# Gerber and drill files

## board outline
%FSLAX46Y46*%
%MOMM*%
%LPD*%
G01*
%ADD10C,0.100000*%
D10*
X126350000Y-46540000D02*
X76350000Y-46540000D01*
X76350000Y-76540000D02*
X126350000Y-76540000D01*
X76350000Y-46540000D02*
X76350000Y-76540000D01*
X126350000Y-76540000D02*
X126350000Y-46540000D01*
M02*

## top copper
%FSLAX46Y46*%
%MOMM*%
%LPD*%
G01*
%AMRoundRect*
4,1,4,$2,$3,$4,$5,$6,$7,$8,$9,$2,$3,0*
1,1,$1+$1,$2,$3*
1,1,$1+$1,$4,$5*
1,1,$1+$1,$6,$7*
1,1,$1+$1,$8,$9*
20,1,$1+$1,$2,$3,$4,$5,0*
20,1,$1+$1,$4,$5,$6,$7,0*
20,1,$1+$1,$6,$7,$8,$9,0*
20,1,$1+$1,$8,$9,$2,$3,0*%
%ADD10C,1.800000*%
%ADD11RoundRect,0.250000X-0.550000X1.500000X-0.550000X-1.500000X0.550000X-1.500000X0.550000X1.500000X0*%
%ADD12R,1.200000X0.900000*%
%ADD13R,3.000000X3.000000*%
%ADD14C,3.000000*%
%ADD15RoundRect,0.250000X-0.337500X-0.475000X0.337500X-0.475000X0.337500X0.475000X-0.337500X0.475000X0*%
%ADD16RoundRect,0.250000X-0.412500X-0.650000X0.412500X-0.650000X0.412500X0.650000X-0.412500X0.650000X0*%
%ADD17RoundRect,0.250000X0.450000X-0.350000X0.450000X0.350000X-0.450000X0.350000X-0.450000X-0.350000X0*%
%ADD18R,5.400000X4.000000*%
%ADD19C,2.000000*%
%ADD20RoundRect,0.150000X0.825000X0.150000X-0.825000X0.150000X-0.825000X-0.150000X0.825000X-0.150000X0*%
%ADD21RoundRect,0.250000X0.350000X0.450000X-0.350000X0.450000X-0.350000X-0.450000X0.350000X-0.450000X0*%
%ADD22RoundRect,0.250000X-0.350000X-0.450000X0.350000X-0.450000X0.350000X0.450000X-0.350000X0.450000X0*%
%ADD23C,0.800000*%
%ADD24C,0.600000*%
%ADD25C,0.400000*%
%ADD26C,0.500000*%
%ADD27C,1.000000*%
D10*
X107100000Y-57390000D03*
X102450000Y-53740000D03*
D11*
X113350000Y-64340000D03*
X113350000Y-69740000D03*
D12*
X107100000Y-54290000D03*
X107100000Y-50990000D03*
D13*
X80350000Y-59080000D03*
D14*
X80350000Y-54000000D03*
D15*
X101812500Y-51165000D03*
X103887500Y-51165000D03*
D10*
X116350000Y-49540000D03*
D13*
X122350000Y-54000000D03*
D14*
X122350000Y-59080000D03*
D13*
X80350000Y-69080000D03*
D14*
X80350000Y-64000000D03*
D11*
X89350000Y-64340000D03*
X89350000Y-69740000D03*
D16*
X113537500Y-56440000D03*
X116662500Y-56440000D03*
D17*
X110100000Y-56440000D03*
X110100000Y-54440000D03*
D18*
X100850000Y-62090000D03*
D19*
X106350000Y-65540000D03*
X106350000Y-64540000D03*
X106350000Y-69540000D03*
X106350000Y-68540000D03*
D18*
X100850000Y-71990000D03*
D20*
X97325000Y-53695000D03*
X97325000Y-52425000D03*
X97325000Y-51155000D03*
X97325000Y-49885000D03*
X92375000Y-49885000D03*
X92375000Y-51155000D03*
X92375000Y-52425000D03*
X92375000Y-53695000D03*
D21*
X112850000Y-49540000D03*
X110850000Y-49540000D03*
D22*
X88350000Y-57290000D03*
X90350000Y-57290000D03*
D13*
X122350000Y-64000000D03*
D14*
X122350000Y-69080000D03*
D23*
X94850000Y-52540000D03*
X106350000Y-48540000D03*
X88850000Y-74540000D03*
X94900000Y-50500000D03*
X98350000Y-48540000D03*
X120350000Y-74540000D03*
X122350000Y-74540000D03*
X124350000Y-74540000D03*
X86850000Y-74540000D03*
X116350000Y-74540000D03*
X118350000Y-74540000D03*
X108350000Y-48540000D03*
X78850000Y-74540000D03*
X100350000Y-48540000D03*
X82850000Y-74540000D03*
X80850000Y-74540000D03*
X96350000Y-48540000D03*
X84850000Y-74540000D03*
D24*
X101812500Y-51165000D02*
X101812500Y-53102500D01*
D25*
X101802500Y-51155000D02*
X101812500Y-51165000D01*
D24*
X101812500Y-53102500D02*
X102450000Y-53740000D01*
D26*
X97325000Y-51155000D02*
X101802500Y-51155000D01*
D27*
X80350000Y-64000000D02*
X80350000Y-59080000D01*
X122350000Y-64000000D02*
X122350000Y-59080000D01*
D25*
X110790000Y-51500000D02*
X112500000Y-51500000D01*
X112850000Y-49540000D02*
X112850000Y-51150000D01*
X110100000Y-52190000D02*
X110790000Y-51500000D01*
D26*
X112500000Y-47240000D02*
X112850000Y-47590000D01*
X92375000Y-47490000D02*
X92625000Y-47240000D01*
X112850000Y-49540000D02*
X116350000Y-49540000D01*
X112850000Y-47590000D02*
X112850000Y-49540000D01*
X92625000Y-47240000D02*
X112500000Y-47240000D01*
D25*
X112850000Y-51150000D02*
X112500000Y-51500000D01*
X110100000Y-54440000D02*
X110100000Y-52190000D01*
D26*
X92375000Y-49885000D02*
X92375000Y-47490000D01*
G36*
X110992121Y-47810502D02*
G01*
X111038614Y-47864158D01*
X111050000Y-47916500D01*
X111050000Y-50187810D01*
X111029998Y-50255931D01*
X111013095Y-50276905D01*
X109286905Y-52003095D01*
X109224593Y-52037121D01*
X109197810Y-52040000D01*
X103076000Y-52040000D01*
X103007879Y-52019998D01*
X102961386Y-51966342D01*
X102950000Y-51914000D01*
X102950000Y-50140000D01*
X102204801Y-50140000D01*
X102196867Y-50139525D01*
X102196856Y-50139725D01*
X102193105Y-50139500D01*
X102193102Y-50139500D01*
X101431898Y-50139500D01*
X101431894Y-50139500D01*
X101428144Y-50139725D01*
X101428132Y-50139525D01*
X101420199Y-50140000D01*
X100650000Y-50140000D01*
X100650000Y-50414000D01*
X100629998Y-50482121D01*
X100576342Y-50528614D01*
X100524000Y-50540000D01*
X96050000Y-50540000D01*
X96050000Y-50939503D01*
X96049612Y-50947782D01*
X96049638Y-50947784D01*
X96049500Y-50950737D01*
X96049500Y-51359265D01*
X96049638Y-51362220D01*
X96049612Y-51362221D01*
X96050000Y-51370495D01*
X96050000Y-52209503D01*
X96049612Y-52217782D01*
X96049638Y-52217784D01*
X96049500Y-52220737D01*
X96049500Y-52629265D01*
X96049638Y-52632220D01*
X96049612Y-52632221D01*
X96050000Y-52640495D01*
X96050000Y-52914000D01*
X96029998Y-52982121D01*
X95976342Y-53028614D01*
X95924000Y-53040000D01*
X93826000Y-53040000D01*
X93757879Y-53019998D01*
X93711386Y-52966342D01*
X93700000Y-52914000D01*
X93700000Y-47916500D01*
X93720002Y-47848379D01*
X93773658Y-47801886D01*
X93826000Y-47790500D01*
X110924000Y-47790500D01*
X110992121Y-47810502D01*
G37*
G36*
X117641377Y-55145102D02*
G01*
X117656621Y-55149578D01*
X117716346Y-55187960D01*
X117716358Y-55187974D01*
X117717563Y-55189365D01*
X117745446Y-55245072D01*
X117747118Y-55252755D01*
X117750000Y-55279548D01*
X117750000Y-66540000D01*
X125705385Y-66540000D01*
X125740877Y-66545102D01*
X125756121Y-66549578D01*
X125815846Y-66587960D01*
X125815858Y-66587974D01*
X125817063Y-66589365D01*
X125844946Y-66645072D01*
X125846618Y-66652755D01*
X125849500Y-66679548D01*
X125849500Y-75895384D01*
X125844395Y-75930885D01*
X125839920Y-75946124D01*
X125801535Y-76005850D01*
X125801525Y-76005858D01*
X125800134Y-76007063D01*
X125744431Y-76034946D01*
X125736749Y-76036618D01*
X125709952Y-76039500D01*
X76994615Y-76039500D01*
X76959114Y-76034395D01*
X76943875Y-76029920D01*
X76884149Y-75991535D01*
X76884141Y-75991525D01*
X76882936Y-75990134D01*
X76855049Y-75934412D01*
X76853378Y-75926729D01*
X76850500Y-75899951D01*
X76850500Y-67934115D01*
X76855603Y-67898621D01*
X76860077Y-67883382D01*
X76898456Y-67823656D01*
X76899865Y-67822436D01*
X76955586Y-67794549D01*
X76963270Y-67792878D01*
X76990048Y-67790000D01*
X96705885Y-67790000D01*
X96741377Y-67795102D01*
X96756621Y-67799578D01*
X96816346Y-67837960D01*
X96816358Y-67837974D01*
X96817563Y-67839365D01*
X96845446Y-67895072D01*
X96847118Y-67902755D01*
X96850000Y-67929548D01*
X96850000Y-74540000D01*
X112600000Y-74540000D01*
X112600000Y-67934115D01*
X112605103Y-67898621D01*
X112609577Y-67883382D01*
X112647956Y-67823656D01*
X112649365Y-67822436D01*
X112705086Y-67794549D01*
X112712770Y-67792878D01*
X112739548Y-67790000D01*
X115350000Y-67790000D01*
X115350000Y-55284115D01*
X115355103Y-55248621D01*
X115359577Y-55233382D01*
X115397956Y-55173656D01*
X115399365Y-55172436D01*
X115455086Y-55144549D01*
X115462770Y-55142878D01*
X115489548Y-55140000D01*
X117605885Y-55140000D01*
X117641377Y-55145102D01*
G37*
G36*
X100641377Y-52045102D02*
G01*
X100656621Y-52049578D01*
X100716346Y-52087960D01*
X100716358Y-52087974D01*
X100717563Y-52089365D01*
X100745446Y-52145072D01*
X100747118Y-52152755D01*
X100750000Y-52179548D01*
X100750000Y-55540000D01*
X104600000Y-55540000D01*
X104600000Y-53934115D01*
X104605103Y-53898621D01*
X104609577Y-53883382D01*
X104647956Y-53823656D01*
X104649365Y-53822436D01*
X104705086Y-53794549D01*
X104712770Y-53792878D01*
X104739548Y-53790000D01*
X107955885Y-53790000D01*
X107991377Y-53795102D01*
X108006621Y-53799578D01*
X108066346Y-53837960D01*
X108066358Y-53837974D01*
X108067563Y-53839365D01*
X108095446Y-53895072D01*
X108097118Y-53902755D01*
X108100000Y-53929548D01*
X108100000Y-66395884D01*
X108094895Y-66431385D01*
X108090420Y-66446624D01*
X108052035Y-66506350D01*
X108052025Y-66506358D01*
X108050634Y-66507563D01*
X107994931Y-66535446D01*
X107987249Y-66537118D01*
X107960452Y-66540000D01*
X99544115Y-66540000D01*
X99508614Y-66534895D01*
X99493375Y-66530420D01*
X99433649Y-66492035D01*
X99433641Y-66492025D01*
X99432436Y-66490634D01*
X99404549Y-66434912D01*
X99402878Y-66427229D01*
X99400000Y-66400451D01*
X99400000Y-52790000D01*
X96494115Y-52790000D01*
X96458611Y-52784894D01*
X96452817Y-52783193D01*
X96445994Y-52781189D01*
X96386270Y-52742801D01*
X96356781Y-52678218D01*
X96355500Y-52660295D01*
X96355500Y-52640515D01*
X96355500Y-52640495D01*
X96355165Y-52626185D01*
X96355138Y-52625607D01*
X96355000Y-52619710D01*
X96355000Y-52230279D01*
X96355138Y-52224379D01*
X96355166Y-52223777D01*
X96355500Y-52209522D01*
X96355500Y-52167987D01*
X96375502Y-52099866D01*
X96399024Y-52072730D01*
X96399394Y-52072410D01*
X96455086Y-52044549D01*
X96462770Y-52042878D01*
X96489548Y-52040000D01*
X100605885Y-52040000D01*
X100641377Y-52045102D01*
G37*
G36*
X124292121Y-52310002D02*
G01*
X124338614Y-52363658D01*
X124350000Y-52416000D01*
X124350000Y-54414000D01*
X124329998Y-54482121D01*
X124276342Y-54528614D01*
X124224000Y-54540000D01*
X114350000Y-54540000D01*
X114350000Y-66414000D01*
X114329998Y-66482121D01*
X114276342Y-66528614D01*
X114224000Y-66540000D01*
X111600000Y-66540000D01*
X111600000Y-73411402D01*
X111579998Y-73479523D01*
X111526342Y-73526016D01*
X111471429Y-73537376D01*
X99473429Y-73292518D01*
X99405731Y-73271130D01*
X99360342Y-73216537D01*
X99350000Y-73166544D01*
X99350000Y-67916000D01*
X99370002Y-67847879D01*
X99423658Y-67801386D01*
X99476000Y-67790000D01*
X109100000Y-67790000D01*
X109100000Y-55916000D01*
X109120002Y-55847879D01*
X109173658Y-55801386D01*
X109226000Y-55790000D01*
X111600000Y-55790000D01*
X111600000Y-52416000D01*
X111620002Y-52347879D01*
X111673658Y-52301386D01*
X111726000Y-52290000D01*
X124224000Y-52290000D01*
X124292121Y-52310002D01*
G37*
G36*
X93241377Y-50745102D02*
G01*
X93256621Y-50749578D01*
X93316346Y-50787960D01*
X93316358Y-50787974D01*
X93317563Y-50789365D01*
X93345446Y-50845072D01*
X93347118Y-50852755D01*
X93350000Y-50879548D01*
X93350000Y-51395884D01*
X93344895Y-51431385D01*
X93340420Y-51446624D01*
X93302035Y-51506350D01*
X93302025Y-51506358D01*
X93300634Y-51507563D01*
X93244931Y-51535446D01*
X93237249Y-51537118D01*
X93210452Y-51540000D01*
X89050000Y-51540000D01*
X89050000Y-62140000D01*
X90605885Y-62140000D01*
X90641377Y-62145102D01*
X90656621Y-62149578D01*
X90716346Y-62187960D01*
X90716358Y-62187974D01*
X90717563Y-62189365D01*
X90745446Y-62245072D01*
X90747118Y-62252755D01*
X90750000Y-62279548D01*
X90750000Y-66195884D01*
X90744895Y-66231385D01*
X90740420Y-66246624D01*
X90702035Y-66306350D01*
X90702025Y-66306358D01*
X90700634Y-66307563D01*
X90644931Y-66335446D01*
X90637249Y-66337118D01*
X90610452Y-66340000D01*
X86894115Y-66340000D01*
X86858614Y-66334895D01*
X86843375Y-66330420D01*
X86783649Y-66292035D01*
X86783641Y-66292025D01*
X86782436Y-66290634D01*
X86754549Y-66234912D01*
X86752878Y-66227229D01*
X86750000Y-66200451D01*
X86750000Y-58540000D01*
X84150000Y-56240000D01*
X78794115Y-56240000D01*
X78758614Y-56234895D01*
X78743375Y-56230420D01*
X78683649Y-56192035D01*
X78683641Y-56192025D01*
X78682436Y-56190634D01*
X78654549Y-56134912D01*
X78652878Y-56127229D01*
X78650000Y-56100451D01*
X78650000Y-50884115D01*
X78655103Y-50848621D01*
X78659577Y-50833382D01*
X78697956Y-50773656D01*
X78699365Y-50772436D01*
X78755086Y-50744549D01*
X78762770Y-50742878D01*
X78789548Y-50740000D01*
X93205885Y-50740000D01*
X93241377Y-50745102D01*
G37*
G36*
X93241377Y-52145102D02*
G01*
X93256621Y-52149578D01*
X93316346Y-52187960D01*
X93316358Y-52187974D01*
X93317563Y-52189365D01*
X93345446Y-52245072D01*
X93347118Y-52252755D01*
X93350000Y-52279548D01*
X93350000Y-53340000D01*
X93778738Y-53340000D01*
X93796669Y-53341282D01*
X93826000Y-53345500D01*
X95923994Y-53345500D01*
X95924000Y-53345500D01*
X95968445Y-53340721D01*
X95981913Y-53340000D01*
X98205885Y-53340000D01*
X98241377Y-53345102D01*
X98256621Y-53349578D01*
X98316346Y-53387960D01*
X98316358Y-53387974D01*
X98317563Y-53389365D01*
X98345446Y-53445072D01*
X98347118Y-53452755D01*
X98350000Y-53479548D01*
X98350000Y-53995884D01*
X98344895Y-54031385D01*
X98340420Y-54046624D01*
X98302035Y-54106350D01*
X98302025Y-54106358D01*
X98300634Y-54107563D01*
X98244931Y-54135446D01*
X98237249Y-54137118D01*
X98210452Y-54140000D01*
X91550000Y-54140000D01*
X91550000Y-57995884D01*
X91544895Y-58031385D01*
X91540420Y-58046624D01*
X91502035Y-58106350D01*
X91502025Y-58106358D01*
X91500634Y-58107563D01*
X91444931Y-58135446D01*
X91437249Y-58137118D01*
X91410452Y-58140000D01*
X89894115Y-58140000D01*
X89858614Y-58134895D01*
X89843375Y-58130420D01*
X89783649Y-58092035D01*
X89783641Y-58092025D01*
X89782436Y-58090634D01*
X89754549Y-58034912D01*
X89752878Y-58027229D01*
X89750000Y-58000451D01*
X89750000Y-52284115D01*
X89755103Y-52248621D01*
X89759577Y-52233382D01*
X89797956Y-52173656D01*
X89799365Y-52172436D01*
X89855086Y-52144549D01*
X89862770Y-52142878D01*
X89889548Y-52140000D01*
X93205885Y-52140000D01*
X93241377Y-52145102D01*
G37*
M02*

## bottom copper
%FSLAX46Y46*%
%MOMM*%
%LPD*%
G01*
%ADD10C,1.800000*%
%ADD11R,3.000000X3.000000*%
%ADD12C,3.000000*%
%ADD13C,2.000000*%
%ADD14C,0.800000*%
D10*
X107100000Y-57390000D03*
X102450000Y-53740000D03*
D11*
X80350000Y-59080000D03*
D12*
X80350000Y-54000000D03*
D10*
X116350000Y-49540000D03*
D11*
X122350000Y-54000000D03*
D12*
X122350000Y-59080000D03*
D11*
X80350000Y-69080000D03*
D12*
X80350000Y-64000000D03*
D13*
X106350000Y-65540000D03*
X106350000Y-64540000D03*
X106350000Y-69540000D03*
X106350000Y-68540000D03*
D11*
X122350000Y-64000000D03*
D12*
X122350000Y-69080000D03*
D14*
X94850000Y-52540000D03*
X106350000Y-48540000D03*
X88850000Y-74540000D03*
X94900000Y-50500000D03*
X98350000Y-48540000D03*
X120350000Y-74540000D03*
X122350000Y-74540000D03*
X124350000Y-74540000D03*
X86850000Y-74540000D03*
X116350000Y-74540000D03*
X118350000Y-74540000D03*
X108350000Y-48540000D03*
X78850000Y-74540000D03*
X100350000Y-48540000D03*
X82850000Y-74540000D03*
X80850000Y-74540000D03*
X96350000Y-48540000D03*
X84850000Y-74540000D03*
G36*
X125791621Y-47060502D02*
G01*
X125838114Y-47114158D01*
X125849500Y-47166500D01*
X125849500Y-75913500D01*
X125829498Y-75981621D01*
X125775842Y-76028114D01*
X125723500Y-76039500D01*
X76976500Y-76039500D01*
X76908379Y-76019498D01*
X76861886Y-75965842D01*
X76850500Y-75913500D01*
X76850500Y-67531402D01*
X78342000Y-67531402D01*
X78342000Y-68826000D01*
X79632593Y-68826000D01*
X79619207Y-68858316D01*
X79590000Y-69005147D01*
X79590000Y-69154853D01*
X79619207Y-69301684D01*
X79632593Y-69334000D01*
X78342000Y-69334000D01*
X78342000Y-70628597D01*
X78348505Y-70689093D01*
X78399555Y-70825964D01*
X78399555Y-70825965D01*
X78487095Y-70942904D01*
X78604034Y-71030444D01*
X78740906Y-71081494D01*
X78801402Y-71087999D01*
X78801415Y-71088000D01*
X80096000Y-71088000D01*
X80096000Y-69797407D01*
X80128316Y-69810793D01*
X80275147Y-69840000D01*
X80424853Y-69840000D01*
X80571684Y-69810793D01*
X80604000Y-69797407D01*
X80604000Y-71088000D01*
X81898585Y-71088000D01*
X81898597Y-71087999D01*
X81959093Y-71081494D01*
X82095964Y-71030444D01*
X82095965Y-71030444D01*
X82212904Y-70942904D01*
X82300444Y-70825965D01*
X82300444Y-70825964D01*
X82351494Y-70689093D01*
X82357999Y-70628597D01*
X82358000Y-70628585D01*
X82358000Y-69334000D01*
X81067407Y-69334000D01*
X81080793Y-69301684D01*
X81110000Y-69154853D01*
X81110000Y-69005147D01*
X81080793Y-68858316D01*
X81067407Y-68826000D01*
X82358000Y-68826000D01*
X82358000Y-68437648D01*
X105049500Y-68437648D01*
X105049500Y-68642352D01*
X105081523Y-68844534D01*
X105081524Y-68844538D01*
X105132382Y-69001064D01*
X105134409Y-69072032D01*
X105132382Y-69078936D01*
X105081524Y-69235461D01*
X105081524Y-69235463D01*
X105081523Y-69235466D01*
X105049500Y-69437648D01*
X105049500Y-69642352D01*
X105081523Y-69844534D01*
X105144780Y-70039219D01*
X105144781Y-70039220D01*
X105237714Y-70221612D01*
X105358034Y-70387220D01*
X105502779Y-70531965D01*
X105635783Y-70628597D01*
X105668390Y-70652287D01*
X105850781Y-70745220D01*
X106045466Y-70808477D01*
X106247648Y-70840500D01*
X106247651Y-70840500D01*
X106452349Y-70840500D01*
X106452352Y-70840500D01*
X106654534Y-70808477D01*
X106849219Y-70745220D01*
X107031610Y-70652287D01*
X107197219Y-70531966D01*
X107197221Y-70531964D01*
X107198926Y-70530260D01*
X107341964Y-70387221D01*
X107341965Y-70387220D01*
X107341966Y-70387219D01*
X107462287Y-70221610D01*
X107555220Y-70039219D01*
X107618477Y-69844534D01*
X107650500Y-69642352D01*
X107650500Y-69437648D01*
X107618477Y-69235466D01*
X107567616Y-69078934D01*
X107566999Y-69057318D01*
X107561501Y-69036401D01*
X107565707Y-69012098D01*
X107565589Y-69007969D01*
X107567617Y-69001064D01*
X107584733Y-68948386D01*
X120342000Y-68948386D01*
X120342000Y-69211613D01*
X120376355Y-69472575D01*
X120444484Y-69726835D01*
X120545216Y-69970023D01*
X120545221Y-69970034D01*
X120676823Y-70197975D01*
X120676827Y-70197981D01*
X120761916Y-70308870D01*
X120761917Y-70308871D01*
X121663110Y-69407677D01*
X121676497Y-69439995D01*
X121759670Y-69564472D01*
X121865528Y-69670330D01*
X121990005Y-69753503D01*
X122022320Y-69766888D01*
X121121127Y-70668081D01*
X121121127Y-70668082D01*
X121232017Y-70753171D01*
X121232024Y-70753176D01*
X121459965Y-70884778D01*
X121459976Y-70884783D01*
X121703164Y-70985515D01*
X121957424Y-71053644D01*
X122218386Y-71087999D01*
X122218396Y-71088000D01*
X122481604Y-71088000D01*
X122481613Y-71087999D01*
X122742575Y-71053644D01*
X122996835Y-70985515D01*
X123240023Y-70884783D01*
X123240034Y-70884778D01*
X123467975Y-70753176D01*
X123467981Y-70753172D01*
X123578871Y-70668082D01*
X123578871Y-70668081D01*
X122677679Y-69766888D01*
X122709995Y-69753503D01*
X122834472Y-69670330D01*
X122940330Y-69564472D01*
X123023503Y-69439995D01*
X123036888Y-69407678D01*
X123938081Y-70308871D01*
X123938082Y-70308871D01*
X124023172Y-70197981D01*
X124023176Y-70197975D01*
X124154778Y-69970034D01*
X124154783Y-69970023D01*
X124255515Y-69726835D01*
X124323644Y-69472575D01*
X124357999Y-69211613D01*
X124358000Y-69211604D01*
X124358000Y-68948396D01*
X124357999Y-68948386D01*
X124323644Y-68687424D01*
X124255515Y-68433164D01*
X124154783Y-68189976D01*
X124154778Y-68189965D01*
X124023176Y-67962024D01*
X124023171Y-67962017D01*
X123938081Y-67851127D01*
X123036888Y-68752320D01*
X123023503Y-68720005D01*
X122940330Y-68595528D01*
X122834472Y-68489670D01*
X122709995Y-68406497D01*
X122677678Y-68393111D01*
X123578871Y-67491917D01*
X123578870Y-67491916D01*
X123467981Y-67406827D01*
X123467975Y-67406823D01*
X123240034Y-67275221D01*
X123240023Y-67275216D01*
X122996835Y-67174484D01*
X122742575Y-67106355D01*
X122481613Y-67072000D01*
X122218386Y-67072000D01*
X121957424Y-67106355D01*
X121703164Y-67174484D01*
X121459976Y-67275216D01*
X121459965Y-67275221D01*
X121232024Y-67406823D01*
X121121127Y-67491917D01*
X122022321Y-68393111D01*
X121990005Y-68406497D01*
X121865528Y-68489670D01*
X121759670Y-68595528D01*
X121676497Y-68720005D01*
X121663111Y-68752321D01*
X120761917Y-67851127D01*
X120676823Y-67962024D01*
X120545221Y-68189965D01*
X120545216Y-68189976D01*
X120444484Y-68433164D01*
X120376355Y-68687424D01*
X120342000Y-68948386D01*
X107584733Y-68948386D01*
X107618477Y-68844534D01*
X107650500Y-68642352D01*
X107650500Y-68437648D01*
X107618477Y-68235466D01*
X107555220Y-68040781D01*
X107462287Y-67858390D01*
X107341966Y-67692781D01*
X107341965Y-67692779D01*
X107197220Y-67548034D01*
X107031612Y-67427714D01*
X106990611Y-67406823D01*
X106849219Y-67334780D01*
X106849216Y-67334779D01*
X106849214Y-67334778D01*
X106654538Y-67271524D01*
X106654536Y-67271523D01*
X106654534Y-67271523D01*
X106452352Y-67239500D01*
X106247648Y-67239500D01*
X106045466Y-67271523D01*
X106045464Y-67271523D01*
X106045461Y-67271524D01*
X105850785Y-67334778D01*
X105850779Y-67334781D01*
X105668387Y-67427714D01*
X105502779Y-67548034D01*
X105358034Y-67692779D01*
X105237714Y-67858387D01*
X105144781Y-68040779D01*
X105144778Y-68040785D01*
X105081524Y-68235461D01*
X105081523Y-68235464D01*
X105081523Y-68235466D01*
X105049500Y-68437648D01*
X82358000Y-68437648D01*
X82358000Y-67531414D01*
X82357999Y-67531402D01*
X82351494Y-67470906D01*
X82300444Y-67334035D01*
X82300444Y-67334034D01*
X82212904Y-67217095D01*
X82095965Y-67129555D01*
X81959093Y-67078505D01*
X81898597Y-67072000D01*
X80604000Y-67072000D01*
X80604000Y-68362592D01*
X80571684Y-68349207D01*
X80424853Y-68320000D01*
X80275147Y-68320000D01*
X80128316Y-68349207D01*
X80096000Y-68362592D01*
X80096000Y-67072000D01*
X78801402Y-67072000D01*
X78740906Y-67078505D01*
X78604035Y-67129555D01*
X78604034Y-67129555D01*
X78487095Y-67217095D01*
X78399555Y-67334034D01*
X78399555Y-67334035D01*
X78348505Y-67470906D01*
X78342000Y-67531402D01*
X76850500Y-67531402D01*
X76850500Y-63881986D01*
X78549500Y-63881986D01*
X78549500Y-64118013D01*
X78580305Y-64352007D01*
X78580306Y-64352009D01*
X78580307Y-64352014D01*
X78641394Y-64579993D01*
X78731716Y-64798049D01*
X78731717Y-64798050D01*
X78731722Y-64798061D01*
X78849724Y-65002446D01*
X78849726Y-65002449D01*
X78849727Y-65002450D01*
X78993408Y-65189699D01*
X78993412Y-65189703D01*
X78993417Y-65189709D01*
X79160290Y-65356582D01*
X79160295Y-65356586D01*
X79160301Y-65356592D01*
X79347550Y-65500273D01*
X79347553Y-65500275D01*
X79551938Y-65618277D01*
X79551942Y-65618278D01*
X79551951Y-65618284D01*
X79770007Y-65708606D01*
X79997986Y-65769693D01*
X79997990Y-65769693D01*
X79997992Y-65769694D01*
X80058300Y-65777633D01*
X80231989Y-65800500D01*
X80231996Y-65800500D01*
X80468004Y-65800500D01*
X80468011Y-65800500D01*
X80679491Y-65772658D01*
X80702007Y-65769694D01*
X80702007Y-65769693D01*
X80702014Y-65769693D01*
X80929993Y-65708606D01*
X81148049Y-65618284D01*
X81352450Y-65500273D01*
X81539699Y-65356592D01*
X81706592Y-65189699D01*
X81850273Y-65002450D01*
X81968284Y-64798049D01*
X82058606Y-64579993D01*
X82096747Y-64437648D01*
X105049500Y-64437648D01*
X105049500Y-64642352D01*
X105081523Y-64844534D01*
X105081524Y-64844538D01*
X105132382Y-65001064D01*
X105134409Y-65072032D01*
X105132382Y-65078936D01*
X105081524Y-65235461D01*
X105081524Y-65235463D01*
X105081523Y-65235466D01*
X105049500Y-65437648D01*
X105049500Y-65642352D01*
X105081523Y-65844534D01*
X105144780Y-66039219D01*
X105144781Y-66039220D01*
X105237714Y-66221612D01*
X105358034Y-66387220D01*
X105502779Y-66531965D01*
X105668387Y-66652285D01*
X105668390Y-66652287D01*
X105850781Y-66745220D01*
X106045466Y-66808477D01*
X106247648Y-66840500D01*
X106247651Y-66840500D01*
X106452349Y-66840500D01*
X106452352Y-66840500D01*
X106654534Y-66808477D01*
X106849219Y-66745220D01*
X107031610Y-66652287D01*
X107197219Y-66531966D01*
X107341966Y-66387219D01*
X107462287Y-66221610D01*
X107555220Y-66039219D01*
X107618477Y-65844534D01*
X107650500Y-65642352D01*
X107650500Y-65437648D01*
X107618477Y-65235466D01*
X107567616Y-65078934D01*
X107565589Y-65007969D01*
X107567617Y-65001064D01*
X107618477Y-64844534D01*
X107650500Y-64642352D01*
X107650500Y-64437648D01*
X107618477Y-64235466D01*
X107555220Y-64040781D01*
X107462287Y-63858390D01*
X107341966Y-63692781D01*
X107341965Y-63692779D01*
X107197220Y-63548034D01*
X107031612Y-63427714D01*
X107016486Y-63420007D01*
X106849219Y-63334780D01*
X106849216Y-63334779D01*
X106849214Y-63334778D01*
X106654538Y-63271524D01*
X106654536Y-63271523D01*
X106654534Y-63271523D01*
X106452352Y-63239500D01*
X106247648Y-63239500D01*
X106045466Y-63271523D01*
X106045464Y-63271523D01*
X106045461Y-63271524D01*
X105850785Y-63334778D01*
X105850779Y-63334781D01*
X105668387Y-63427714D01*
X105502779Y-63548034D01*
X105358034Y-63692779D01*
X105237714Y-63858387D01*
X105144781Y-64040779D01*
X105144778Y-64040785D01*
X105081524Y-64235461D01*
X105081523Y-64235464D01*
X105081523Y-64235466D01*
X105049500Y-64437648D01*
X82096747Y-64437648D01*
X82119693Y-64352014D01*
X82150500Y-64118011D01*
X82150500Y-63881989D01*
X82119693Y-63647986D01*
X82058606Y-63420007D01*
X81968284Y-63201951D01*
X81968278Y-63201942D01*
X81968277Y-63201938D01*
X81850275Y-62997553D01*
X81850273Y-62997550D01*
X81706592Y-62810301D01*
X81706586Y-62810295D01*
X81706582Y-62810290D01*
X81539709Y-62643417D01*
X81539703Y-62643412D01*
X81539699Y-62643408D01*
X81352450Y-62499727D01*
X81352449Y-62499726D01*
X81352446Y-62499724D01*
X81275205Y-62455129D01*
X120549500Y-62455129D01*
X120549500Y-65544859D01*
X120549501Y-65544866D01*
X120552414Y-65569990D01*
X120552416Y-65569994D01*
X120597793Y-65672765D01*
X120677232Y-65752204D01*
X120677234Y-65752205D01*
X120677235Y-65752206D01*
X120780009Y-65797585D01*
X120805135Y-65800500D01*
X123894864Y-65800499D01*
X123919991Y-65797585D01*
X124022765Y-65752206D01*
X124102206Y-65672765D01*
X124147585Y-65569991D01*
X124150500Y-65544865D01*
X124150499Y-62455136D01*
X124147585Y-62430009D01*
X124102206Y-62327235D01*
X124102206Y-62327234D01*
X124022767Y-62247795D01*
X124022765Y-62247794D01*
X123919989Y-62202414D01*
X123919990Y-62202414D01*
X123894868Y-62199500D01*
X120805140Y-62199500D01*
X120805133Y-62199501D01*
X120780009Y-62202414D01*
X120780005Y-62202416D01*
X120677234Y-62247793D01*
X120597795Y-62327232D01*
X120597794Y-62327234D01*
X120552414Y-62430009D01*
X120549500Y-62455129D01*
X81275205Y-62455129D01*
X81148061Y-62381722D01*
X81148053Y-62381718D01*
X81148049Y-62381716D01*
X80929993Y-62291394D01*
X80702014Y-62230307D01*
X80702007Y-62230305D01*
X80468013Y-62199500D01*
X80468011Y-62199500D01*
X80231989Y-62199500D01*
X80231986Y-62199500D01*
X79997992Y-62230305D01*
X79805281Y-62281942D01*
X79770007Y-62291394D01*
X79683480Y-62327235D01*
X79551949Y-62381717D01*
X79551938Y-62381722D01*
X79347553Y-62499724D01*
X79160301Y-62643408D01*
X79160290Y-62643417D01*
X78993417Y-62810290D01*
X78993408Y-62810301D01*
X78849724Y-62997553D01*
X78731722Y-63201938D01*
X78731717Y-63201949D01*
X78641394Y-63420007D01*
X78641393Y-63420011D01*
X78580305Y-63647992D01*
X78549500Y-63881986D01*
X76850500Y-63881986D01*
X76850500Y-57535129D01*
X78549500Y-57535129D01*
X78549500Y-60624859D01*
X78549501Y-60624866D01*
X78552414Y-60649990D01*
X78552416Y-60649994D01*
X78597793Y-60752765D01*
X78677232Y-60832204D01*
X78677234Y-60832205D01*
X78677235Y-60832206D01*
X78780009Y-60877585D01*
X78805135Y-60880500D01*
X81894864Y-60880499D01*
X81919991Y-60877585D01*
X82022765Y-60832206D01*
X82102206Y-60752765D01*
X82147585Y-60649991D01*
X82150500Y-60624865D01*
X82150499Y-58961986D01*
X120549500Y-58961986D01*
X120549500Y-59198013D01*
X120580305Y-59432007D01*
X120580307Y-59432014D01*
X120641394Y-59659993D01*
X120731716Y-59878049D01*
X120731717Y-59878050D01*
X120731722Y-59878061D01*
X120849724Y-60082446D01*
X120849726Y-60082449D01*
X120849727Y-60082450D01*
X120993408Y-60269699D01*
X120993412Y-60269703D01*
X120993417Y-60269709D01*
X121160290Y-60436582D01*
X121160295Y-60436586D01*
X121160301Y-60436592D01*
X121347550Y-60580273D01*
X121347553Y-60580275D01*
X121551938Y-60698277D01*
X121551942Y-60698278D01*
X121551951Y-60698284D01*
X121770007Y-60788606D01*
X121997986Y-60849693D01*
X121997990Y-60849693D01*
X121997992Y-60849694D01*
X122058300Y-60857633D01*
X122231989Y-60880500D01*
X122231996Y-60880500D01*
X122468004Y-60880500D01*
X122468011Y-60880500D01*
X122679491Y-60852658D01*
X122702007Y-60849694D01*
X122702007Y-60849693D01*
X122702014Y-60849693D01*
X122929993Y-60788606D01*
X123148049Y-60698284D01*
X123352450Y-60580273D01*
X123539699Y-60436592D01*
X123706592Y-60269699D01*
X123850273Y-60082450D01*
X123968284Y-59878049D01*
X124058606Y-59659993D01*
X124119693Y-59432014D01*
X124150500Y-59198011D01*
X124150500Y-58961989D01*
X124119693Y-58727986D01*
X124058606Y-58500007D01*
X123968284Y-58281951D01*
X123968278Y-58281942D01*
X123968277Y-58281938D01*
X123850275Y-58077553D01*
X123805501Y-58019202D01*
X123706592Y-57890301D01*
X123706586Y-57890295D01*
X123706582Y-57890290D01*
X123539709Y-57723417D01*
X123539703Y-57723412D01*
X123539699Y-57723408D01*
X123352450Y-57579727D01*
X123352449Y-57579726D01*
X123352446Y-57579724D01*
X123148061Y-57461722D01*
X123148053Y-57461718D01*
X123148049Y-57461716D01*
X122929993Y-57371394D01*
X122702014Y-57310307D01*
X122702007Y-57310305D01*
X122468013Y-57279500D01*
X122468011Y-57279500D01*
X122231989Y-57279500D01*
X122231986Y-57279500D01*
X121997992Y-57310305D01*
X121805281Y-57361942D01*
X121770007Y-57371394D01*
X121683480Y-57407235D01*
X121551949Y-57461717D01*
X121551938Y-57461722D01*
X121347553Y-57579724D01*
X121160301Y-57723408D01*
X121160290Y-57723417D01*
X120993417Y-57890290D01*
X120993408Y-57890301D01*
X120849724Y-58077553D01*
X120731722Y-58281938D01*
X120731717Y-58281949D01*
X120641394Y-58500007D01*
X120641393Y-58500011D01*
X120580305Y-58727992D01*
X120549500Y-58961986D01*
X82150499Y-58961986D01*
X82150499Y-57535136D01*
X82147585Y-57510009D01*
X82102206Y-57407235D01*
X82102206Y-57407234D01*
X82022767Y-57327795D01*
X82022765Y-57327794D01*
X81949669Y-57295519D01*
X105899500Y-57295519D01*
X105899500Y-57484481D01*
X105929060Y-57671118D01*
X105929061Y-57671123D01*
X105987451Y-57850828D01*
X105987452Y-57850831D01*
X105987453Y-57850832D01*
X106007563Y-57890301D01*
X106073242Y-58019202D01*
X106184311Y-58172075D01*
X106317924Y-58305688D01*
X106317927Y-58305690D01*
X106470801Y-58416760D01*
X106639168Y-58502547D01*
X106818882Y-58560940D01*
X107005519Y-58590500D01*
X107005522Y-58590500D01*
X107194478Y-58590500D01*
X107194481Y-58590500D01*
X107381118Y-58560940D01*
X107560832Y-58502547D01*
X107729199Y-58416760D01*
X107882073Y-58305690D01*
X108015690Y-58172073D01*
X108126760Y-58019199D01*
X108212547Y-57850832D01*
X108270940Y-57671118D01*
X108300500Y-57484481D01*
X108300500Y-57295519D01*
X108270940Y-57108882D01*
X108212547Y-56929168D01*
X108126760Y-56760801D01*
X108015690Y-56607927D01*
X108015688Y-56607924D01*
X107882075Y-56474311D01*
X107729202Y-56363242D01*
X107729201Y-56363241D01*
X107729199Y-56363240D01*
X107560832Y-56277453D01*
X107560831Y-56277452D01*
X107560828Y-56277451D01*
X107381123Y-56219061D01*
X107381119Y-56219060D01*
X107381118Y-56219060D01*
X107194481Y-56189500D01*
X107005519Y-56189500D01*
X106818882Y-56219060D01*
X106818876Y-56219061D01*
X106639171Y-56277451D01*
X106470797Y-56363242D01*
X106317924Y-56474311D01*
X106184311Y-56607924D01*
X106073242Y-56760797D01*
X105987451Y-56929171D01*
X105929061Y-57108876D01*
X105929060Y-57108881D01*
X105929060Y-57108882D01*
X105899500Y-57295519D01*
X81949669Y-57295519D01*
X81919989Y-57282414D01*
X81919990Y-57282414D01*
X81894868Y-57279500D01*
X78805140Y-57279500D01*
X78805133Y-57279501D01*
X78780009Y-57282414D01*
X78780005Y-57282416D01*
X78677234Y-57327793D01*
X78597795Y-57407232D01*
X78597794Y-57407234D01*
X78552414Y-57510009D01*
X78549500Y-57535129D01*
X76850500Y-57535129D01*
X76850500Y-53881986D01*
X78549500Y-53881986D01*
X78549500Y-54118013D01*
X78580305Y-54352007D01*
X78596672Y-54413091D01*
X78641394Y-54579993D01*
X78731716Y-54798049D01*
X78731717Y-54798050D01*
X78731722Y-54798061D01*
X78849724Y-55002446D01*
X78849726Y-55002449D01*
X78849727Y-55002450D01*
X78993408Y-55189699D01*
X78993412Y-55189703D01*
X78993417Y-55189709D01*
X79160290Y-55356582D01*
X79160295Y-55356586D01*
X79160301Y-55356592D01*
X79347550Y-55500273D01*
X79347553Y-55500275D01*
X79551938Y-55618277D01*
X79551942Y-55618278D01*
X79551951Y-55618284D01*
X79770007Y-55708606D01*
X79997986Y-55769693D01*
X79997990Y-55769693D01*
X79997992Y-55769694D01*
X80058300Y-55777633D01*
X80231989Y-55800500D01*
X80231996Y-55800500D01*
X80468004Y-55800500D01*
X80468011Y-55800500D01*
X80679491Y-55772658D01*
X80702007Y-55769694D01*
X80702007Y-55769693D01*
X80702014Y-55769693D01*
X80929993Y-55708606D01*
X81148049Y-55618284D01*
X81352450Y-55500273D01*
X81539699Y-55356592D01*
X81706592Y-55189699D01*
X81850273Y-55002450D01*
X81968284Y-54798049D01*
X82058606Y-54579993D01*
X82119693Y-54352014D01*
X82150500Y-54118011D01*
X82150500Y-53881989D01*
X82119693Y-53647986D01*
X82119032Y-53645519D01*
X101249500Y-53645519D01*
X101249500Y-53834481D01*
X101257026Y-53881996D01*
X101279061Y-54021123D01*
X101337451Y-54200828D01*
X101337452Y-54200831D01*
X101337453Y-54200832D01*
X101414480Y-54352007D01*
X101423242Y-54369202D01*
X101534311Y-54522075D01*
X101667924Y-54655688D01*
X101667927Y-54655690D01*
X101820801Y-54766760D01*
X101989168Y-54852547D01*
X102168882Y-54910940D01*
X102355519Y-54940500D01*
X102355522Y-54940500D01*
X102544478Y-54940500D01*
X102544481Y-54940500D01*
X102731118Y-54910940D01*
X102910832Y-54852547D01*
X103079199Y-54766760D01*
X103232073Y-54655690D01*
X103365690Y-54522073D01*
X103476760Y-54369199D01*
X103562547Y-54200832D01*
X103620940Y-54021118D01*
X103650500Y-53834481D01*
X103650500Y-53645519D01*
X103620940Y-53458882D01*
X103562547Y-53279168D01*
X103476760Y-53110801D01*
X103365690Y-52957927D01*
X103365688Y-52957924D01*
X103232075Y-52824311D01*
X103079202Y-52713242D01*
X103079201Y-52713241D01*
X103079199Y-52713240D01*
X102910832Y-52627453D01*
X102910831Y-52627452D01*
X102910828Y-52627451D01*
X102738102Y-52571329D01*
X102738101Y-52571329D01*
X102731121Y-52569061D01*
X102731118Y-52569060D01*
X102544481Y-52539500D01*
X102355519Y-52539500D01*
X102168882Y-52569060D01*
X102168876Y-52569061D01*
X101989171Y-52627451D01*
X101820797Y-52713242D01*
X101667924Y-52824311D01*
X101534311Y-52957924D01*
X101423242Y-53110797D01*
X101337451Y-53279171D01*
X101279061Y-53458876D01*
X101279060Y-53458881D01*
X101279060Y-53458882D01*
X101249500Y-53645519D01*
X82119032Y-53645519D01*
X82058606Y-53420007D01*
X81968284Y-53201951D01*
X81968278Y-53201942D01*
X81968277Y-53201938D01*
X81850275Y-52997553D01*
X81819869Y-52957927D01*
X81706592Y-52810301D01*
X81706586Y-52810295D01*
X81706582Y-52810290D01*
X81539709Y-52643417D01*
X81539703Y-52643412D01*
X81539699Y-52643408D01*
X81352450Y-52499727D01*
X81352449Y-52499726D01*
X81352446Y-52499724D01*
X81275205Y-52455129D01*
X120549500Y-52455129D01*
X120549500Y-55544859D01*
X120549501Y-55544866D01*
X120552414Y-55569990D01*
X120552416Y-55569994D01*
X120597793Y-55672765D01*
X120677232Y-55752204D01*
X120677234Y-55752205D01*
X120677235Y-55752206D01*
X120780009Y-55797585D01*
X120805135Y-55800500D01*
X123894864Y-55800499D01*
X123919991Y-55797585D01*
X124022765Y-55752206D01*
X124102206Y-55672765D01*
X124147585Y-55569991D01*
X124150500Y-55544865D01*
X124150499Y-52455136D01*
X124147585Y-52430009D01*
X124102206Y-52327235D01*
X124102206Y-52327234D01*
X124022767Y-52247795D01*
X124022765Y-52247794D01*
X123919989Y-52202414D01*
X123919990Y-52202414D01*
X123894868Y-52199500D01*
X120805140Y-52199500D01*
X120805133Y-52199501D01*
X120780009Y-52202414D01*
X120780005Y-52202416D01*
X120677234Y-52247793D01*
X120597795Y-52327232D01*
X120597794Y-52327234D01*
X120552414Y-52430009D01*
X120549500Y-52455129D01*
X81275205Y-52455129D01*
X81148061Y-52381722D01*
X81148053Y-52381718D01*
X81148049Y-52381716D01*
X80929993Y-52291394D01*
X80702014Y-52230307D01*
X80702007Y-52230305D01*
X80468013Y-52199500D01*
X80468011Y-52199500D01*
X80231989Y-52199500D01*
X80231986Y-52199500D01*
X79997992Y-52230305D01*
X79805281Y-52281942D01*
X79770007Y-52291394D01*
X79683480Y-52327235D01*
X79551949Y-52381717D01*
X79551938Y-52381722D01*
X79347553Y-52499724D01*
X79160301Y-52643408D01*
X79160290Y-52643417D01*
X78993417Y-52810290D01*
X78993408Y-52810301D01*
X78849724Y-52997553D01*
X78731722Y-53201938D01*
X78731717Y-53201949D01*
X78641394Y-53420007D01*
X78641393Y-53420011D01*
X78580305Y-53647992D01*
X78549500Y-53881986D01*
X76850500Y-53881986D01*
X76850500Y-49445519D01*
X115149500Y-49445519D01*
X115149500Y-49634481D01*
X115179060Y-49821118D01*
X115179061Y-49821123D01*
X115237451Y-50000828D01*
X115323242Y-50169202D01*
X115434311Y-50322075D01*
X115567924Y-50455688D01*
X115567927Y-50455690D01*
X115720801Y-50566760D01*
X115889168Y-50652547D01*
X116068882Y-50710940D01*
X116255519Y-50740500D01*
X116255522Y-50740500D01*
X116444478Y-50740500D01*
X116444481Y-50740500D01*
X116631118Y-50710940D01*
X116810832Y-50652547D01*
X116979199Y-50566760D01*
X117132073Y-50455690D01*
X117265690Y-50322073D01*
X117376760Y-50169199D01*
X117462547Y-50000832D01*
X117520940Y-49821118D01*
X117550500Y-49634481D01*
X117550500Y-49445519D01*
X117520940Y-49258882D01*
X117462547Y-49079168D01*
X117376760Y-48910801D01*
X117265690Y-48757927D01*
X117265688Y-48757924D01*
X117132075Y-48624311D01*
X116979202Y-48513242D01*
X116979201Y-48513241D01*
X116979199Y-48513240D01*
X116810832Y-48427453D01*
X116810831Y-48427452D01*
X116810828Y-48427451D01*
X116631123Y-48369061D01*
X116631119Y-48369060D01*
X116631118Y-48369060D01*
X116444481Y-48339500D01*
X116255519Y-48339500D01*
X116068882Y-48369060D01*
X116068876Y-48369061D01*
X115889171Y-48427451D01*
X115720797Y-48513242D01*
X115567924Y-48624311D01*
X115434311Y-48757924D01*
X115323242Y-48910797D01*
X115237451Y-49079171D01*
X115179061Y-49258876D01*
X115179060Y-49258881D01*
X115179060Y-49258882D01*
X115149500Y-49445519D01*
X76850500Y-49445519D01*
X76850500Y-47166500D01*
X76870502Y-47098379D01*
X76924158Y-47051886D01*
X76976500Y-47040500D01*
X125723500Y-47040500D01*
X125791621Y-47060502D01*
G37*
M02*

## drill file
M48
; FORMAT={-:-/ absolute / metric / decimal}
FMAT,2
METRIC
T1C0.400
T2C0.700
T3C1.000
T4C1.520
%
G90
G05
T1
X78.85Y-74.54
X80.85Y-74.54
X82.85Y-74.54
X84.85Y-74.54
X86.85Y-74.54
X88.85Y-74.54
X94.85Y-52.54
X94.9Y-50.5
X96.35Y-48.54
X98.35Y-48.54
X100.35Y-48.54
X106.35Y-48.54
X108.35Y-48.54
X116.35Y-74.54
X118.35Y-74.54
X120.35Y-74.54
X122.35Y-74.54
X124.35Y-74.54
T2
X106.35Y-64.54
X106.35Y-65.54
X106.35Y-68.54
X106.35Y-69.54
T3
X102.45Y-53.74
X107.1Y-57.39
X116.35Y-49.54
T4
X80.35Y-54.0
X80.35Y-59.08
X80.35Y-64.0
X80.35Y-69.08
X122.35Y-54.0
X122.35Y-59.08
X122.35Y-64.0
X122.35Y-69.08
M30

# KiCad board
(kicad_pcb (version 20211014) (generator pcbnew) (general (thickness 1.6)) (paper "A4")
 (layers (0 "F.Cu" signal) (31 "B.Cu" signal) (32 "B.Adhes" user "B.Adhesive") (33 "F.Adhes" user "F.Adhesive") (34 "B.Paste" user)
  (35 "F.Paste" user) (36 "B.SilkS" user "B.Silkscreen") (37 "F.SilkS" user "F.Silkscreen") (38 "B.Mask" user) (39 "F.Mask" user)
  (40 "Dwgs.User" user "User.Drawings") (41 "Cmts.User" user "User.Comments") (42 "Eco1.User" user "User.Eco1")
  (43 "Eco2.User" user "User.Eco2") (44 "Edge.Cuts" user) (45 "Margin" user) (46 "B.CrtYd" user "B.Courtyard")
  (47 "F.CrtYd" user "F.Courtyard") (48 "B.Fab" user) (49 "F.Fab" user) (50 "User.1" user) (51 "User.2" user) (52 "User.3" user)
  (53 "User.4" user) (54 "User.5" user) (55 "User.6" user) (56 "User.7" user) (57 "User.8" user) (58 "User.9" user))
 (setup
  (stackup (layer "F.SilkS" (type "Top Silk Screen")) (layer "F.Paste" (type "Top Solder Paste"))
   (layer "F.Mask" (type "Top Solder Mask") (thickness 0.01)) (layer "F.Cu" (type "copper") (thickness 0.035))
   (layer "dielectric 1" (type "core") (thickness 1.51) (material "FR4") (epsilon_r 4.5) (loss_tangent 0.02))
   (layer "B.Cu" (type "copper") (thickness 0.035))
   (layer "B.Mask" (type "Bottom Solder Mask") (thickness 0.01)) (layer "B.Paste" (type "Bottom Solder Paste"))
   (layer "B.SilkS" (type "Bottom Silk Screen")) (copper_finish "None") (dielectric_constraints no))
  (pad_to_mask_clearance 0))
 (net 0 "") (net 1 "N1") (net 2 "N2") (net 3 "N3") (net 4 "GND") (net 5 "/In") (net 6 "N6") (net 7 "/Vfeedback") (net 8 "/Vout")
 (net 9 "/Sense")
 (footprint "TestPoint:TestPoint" (layer "F.Cu") (at 107.1 57.39)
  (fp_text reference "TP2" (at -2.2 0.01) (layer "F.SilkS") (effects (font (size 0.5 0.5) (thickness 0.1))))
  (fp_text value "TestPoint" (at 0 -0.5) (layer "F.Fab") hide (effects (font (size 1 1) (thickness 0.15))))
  (pad "1" thru_hole circle locked (at 0 0) (size 1.8 1.8) (drill 1) (layers *.Cu *.Mask) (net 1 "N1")))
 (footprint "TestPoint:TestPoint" (layer "F.Cu") (at 102.45 53.74)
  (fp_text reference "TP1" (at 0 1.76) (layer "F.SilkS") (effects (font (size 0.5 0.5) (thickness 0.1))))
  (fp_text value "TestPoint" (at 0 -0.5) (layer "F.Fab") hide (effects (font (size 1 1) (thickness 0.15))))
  (pad "1" thru_hole circle locked (at 0 0) (size 1.8 1.8) (drill 1) (layers *.Cu *.Mask) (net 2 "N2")))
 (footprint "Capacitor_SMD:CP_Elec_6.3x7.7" (layer "F.Cu") (at 113.35 67.04 -90)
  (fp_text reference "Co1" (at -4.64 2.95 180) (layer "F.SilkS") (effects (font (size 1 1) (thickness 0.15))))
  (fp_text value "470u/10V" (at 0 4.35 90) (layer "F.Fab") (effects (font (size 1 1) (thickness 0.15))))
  (pad "1" smd roundrect (at -2.7 0 270) (size 3.5 1.6) (layers "F.Cu" "F.Paste" "F.Mask") (roundrect_rratio 0.15625) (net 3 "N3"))
  (pad "2" smd roundrect (at 2.7 0 270) (size 3.5 1.6) (layers "F.Cu" "F.Paste" "F.Mask") (roundrect_rratio 0.15625) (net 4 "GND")))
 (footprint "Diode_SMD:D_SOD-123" (layer "F.Cu") (at 107.1 52.64 90)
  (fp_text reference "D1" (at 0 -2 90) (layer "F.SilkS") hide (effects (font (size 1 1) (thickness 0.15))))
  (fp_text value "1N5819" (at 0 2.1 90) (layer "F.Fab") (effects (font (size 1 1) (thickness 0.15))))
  (pad "1" smd rect (at -1.65 0 90) (size 0.9 1.2) (layers "F.Cu" "F.Paste" "F.Mask") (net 1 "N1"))
  (pad "2" smd rect (at 1.65 0 90) (size 0.9 1.2) (layers "F.Cu" "F.Paste" "F.Mask") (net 4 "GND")))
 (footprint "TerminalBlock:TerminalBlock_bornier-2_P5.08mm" (layer "F.Cu") (at 80.35 59.08 90)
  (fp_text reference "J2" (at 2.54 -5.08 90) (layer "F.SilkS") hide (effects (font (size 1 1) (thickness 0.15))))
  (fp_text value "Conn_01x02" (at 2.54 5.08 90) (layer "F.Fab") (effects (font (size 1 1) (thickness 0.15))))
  (pad "1" thru_hole rect (at 0 0 90) (size 3 3) (drill 1.52) (layers *.Cu *.Mask) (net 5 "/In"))
  (pad "2" thru_hole circle (at 5.08 0 90) (size 3 3) (drill 1.52) (layers *.Cu *.Mask) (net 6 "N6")))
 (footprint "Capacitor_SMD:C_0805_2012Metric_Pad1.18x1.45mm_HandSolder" (layer "F.Cu") (at 102.85 51.165)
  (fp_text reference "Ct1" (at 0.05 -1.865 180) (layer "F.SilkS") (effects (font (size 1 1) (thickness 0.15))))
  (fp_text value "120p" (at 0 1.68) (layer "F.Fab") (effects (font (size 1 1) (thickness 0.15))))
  (pad "1" smd roundrect (at -1.0375 0) (size 1.175 1.45) (layers "F.Cu" "F.Paste" "F.Mask") (roundrect_rratio 0.2127659574) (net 2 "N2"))
  (pad "2" smd roundrect (at 1.0375 0) (size 1.175 1.45) (layers "F.Cu" "F.Paste" "F.Mask") (roundrect_rratio 0.2127659574) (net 4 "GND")))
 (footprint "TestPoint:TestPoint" (layer "F.Cu") (at 116.35 49.54)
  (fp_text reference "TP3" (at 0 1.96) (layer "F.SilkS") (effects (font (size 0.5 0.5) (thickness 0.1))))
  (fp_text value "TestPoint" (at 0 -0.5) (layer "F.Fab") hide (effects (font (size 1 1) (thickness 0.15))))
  (pad "1" thru_hole circle locked (at 0 0) (size 1.8 1.8) (drill 1) (layers *.Cu *.Mask) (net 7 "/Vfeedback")))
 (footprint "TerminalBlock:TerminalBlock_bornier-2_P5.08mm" (layer "F.Cu") (at 122.35 54 -90)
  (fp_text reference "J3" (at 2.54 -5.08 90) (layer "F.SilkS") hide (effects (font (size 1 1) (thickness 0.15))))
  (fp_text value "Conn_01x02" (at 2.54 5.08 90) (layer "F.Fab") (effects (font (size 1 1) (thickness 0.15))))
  (pad "1" thru_hole rect (at 0 0 270) (size 3 3) (drill 1.52) (layers *.Cu *.Mask) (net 3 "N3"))
  (pad "2" thru_hole circle (at 5.08 0 270) (size 3 3) (drill 1.52) (layers *.Cu *.Mask) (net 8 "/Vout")))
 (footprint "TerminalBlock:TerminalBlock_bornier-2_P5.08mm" (layer "F.Cu") (at 80.35 69.08 90)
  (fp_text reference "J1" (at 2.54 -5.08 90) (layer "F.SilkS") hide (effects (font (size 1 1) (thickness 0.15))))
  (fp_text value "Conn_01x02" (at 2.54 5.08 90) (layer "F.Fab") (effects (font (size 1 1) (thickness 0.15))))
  (pad "1" thru_hole rect (at 0 0 90) (size 3 3) (drill 1.52) (layers *.Cu *.Mask) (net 4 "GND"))
  (pad "2" thru_hole circle (at 5.08 0 90) (size 3 3) (drill 1.52) (layers *.Cu *.Mask) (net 5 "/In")))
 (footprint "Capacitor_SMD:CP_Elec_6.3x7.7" (layer "F.Cu") (at 89.35 67.04 -90)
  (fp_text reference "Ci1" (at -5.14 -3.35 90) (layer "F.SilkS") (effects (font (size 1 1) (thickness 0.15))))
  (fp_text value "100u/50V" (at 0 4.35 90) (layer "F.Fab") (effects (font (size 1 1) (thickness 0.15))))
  (pad "1" smd roundrect (at -2.7 0 270) (size 3.5 1.6) (layers "F.Cu" "F.Paste" "F.Mask") (roundrect_rratio 0.15625) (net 6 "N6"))
  (pad "2" smd roundrect (at 2.7 0 270) (size 3.5 1.6) (layers "F.Cu" "F.Paste" "F.Mask") (roundrect_rratio 0.15625) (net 4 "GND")))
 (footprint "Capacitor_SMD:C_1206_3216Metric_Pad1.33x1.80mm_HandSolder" (layer "F.Cu") (at 115.1 56.44)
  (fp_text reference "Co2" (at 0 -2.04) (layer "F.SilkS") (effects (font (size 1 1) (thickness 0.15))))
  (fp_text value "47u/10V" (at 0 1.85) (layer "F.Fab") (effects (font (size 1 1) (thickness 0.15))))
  (pad "1" smd roundrect (at -1.5625 0) (size 1.325 1.8) (layers "F.Cu" "F.Paste" "F.Mask") (roundrect_rratio 0.1886792453) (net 3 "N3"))
  (pad "2" smd roundrect (at 1.5625 0) (size 1.325 1.8) (layers "F.Cu" "F.Paste" "F.Mask") (roundrect_rratio 0.1886792453) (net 4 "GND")))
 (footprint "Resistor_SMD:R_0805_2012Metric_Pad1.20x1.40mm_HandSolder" (layer "F.Cu") (at 110.1 55.44 90)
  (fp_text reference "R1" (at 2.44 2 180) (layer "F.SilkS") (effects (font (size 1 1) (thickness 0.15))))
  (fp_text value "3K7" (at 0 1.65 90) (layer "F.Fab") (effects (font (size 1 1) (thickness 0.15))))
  (pad "1" smd roundrect (at -1 0 90) (size 1.2 1.4) (layers "F.Cu" "F.Paste" "F.Mask") (roundrect_rratio 0.2083333333) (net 3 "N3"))
  (pad "2" smd roundrect (at 1 0 90) (size 1.2 1.4) (layers "F.Cu" "F.Paste" "F.Mask") (roundrect_rratio 0.2083333333) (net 7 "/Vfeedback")))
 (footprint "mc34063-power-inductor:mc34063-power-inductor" (layer "F.Cu") (at 100.85 67.04 -90)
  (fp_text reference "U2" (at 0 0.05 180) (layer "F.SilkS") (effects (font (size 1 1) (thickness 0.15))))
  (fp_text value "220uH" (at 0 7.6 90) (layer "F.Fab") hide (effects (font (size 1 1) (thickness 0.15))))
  (pad "1" smd rect (at -4.95 0 270) (size 4 5.4) (layers "F.Cu" "F.Paste" "F.Mask") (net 1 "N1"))
  (pad "1" thru_hole circle (at -1.5 -5.5) (size 2 2) (drill 0.7) (layers *.Cu *.Mask) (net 1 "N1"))
  (pad "1" thru_hole circle (at -2.5 -5.5) (size 2 2) (drill 0.7) (layers *.Cu *.Mask) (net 1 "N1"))
  (pad "2" thru_hole circle (at 2.5 -5.5) (size 2 2) (drill 0.7) (layers *.Cu *.Mask) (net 3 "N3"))
  (pad "2" thru_hole circle (at 1.5 -5.5) (size 2 2) (drill 0.7) (layers *.Cu *.Mask) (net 3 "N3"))
  (pad "2" smd rect (at 4.95 0 270) (size 4 5.4) (layers "F.Cu" "F.Paste" "F.Mask") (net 3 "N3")))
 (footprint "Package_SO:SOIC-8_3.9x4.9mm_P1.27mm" (layer "F.Cu") (at 94.85 51.79 180)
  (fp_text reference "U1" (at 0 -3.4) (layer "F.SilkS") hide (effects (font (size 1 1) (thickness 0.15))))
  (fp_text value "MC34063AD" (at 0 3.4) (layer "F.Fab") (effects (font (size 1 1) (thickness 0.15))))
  (pad "1" smd roundrect (at -2.475 -1.905 180) (size 1.95 0.6) (layers "F.Cu" "F.Paste" "F.Mask") (roundrect_rratio 0.25) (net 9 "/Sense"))
  (pad "2" smd roundrect (at -2.475 -0.635 180) (size 1.95 0.6) (layers "F.Cu" "F.Paste" "F.Mask") (roundrect_rratio 0.25) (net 1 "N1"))
  (pad "3" smd roundrect (at -2.475 0.635 180) (size 1.95 0.6) (layers "F.Cu" "F.Paste" "F.Mask") (roundrect_rratio 0.25) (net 2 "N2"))
  (pad "4" smd roundrect (at -2.475 1.905 180) (size 1.95 0.6) (layers "F.Cu" "F.Paste" "F.Mask") (roundrect_rratio 0.25) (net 4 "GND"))
  (pad "5" smd roundrect (at 2.475 1.905 180) (size 1.95 0.6) (layers "F.Cu" "F.Paste" "F.Mask") (roundrect_rratio 0.25)
   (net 7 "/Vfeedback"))
  (pad "6" smd roundrect (at 2.475 0.635 180) (size 1.95 0.6) (layers "F.Cu" "F.Paste" "F.Mask") (roundrect_rratio 0.25) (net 6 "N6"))
  (pad "7" smd roundrect (at 2.475 -0.635 180) (size 1.95 0.6) (layers "F.Cu" "F.Paste" "F.Mask") (roundrect_rratio 0.25) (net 9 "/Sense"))
  (pad "8" smd roundrect (at 2.475 -1.905 180) (size 1.95 0.6) (layers "F.Cu" "F.Paste" "F.Mask") (roundrect_rratio 0.25) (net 9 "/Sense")))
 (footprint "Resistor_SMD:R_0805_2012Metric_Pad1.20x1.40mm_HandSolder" (layer "F.Cu") (at 111.85 49.54 180)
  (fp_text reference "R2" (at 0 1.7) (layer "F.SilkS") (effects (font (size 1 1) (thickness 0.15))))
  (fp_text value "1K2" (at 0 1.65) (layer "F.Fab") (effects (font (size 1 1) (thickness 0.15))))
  (pad "1" smd roundrect (at -1 0 180) (size 1.2 1.4) (layers "F.Cu" "F.Paste" "F.Mask") (roundrect_rratio 0.2083333333)
   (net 7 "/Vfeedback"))
  (pad "2" smd roundrect (at 1 0 180) (size 1.2 1.4) (layers "F.Cu" "F.Paste" "F.Mask") (roundrect_rratio 0.2083333333) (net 4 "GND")))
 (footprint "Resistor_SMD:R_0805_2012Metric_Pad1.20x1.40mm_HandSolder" (layer "F.Cu") (at 89.35 57.29)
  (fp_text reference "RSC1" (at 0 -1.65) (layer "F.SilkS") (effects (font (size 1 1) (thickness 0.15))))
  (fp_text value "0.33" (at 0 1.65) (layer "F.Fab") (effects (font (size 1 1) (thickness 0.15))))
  (pad "1" smd roundrect (at -1 0) (size 1.2 1.4) (layers "F.Cu" "F.Paste" "F.Mask") (roundrect_rratio 0.2083333333) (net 6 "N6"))
  (pad "2" smd roundrect (at 1 0) (size 1.2 1.4) (layers "F.Cu" "F.Paste" "F.Mask") (roundrect_rratio 0.2083333333) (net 9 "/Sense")))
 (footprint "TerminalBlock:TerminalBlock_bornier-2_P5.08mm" (layer "F.Cu") (at 122.35 64 -90)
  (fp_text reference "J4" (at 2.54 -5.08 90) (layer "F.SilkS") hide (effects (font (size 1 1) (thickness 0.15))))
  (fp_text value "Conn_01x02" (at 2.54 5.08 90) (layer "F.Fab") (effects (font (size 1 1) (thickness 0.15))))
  (pad "1" thru_hole rect (at 0 0 270) (size 3 3) (drill 1.52) (layers *.Cu *.Mask) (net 8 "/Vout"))
  (pad "2" thru_hole circle (at 5.08 0 270) (size 3 3) (drill 1.52) (layers *.Cu *.Mask) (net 4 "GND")))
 (gr_line (start 126.35 46.54) (end 76.35 46.54) (layer "Edge.Cuts") (width 0.1))
 (gr_line (start 76.35 76.54) (end 126.35 76.54) (layer "Edge.Cuts") (width 0.1))
 (gr_line (start 76.35 46.54) (end 76.35 76.54) (layer "Edge.Cuts") (width 0.1))
 (gr_line (start 126.35 76.54) (end 126.35 46.54) (layer "Edge.Cuts") (width 0.1))
 (via (at 94.85 52.54) (size 0.8) (drill 0.4) (layers "F.Cu" "B.Cu") (free) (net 4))
 (via (at 106.35 48.54) (size 0.8) (drill 0.4) (layers "F.Cu" "B.Cu") (free) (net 4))
 (via (at 88.85 74.54) (size 0.8) (drill 0.4) (layers "F.Cu" "B.Cu") (free) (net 4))
 (via (at 94.9 50.5) (size 0.8) (drill 0.4) (layers "F.Cu" "B.Cu") (free) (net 4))
 (via (at 98.35 48.54) (size 0.8) (drill 0.4) (layers "F.Cu" "B.Cu") (free) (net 4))
 (via (at 120.35 74.54) (size 0.8) (drill 0.4) (layers "F.Cu" "B.Cu") (free) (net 4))
 (via (at 122.35 74.54) (size 0.8) (drill 0.4) (layers "F.Cu" "B.Cu") (free) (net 4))
 (via (at 124.35 74.54) (size 0.8) (drill 0.4) (layers "F.Cu" "B.Cu") (free) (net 4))
 (via (at 86.85 74.54) (size 0.8) (drill 0.4) (layers "F.Cu" "B.Cu") (free) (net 4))
 (via (at 116.35 74.54) (size 0.8) (drill 0.4) (layers "F.Cu" "B.Cu") (free) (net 4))
 (via (at 118.35 74.54) (size 0.8) (drill 0.4) (layers "F.Cu" "B.Cu") (free) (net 4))
 (via (at 108.35 48.54) (size 0.8) (drill 0.4) (layers "F.Cu" "B.Cu") (free) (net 4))
 (via (at 78.85 74.54) (size 0.8) (drill 0.4) (layers "F.Cu" "B.Cu") (free) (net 4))
 (via (at 100.35 48.54) (size 0.8) (drill 0.4) (layers "F.Cu" "B.Cu") (free) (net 4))
 (via (at 82.85 74.54) (size 0.8) (drill 0.4) (layers "F.Cu" "B.Cu") (free) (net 4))
 (via (at 80.85 74.54) (size 0.8) (drill 0.4) (layers "F.Cu" "B.Cu") (free) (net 4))
 (via (at 96.35 48.54) (size 0.8) (drill 0.4) (layers "F.Cu" "B.Cu") (free) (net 4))
 (via (at 84.85 74.54) (size 0.8) (drill 0.4) (layers "F.Cu" "B.Cu") (free) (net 4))
 (segment (start 101.8125 51.165) (end 101.8125 53.1025) (width 0.6) (layer "F.Cu") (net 2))
 (segment (start 101.8025 51.155) (end 101.8125 51.165) (width 0.4) (layer "F.Cu") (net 2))
 (segment (start 101.8125 53.1025) (end 102.45 53.74) (width 0.6) (layer "F.Cu") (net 2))
 (segment (start 97.325 51.155) (end 101.8025 51.155) (width 0.5) (layer "F.Cu") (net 2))
 (segment (start 80.35 64) (end 80.35 59.08) (width 1) (layer "F.Cu") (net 5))
 (segment (start 122.35 64) (end 122.35 59.08) (width 1) (layer "F.Cu") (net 8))
 (segment (start 110.79 51.5) (end 112.5 51.5) (width 0.4) (layer "F.Cu") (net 7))
 (segment (start 112.85 49.54) (end 112.85 51.15) (width 0.4) (layer "F.Cu") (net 7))
 (segment (start 110.1 52.19) (end 110.79 51.5) (width 0.4) (layer "F.Cu") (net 7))
 (segment (start 112.5 47.24) (end 112.85 47.59) (width 0.5) (layer "F.Cu") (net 7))
 (segment (start 92.375 47.49) (end 92.625 47.24) (width 0.5) (layer "F.Cu") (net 7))
 (segment (start 112.85 49.54) (end 116.35 49.54) (width 0.5) (layer "F.Cu") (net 7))
 (segment (start 112.85 47.59) (end 112.85 49.54) (width 0.5) (layer "F.Cu") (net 7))
 (segment (start 92.625 47.24) (end 112.5 47.24) (width 0.5) (layer "F.Cu") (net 7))
 (segment (start 112.85 51.15) (end 112.5 51.5) (width 0.4) (layer "F.Cu") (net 7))
 (segment (start 110.1 54.44) (end 110.1 52.19) (width 0.4) (layer "F.Cu") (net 7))
 (segment (start 92.375 49.885) (end 92.375 47.49) (width 0.5) (layer "F.Cu") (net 7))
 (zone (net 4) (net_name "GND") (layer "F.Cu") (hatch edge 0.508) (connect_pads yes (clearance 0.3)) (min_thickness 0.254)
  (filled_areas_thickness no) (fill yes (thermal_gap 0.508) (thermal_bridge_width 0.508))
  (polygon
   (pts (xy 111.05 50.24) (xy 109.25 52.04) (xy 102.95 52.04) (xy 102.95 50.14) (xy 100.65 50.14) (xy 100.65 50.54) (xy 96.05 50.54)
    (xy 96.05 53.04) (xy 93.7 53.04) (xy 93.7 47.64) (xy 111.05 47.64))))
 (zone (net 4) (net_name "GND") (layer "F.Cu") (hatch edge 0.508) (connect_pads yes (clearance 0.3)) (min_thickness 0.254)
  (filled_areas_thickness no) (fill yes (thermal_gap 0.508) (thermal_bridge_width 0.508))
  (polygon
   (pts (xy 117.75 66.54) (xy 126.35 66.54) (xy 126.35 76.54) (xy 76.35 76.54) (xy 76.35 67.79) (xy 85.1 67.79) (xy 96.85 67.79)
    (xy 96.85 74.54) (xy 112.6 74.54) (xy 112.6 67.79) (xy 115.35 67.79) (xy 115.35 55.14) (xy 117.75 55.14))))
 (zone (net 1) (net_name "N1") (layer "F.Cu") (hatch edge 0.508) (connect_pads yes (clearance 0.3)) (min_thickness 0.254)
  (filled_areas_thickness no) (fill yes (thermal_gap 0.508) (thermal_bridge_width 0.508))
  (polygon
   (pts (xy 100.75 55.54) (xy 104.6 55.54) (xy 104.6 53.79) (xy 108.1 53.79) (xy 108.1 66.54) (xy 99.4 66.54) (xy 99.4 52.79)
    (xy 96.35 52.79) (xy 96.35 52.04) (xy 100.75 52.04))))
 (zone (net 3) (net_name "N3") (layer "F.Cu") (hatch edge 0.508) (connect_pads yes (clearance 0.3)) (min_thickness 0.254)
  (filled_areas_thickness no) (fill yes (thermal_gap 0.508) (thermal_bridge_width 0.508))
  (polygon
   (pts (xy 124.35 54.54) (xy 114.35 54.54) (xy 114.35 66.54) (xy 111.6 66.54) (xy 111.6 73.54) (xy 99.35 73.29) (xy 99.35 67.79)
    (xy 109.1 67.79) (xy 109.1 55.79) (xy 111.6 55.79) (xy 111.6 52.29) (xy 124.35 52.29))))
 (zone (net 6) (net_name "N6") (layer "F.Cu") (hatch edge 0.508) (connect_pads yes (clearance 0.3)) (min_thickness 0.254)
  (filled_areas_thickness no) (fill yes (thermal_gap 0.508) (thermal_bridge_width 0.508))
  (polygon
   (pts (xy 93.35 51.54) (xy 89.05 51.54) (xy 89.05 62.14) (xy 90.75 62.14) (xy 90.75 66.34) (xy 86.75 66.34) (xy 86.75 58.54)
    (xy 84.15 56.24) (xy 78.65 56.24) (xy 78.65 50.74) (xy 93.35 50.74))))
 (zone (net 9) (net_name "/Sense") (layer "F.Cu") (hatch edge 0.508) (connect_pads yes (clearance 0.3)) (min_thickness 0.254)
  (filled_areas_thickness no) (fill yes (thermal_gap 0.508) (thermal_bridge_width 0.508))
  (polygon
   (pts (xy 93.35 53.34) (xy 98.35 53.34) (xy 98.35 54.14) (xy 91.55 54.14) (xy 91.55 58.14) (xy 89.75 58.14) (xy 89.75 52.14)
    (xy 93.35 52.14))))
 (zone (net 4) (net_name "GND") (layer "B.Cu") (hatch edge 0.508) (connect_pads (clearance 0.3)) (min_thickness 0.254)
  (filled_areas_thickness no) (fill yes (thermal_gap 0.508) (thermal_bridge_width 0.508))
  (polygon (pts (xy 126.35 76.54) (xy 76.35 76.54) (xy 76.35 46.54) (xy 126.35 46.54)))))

